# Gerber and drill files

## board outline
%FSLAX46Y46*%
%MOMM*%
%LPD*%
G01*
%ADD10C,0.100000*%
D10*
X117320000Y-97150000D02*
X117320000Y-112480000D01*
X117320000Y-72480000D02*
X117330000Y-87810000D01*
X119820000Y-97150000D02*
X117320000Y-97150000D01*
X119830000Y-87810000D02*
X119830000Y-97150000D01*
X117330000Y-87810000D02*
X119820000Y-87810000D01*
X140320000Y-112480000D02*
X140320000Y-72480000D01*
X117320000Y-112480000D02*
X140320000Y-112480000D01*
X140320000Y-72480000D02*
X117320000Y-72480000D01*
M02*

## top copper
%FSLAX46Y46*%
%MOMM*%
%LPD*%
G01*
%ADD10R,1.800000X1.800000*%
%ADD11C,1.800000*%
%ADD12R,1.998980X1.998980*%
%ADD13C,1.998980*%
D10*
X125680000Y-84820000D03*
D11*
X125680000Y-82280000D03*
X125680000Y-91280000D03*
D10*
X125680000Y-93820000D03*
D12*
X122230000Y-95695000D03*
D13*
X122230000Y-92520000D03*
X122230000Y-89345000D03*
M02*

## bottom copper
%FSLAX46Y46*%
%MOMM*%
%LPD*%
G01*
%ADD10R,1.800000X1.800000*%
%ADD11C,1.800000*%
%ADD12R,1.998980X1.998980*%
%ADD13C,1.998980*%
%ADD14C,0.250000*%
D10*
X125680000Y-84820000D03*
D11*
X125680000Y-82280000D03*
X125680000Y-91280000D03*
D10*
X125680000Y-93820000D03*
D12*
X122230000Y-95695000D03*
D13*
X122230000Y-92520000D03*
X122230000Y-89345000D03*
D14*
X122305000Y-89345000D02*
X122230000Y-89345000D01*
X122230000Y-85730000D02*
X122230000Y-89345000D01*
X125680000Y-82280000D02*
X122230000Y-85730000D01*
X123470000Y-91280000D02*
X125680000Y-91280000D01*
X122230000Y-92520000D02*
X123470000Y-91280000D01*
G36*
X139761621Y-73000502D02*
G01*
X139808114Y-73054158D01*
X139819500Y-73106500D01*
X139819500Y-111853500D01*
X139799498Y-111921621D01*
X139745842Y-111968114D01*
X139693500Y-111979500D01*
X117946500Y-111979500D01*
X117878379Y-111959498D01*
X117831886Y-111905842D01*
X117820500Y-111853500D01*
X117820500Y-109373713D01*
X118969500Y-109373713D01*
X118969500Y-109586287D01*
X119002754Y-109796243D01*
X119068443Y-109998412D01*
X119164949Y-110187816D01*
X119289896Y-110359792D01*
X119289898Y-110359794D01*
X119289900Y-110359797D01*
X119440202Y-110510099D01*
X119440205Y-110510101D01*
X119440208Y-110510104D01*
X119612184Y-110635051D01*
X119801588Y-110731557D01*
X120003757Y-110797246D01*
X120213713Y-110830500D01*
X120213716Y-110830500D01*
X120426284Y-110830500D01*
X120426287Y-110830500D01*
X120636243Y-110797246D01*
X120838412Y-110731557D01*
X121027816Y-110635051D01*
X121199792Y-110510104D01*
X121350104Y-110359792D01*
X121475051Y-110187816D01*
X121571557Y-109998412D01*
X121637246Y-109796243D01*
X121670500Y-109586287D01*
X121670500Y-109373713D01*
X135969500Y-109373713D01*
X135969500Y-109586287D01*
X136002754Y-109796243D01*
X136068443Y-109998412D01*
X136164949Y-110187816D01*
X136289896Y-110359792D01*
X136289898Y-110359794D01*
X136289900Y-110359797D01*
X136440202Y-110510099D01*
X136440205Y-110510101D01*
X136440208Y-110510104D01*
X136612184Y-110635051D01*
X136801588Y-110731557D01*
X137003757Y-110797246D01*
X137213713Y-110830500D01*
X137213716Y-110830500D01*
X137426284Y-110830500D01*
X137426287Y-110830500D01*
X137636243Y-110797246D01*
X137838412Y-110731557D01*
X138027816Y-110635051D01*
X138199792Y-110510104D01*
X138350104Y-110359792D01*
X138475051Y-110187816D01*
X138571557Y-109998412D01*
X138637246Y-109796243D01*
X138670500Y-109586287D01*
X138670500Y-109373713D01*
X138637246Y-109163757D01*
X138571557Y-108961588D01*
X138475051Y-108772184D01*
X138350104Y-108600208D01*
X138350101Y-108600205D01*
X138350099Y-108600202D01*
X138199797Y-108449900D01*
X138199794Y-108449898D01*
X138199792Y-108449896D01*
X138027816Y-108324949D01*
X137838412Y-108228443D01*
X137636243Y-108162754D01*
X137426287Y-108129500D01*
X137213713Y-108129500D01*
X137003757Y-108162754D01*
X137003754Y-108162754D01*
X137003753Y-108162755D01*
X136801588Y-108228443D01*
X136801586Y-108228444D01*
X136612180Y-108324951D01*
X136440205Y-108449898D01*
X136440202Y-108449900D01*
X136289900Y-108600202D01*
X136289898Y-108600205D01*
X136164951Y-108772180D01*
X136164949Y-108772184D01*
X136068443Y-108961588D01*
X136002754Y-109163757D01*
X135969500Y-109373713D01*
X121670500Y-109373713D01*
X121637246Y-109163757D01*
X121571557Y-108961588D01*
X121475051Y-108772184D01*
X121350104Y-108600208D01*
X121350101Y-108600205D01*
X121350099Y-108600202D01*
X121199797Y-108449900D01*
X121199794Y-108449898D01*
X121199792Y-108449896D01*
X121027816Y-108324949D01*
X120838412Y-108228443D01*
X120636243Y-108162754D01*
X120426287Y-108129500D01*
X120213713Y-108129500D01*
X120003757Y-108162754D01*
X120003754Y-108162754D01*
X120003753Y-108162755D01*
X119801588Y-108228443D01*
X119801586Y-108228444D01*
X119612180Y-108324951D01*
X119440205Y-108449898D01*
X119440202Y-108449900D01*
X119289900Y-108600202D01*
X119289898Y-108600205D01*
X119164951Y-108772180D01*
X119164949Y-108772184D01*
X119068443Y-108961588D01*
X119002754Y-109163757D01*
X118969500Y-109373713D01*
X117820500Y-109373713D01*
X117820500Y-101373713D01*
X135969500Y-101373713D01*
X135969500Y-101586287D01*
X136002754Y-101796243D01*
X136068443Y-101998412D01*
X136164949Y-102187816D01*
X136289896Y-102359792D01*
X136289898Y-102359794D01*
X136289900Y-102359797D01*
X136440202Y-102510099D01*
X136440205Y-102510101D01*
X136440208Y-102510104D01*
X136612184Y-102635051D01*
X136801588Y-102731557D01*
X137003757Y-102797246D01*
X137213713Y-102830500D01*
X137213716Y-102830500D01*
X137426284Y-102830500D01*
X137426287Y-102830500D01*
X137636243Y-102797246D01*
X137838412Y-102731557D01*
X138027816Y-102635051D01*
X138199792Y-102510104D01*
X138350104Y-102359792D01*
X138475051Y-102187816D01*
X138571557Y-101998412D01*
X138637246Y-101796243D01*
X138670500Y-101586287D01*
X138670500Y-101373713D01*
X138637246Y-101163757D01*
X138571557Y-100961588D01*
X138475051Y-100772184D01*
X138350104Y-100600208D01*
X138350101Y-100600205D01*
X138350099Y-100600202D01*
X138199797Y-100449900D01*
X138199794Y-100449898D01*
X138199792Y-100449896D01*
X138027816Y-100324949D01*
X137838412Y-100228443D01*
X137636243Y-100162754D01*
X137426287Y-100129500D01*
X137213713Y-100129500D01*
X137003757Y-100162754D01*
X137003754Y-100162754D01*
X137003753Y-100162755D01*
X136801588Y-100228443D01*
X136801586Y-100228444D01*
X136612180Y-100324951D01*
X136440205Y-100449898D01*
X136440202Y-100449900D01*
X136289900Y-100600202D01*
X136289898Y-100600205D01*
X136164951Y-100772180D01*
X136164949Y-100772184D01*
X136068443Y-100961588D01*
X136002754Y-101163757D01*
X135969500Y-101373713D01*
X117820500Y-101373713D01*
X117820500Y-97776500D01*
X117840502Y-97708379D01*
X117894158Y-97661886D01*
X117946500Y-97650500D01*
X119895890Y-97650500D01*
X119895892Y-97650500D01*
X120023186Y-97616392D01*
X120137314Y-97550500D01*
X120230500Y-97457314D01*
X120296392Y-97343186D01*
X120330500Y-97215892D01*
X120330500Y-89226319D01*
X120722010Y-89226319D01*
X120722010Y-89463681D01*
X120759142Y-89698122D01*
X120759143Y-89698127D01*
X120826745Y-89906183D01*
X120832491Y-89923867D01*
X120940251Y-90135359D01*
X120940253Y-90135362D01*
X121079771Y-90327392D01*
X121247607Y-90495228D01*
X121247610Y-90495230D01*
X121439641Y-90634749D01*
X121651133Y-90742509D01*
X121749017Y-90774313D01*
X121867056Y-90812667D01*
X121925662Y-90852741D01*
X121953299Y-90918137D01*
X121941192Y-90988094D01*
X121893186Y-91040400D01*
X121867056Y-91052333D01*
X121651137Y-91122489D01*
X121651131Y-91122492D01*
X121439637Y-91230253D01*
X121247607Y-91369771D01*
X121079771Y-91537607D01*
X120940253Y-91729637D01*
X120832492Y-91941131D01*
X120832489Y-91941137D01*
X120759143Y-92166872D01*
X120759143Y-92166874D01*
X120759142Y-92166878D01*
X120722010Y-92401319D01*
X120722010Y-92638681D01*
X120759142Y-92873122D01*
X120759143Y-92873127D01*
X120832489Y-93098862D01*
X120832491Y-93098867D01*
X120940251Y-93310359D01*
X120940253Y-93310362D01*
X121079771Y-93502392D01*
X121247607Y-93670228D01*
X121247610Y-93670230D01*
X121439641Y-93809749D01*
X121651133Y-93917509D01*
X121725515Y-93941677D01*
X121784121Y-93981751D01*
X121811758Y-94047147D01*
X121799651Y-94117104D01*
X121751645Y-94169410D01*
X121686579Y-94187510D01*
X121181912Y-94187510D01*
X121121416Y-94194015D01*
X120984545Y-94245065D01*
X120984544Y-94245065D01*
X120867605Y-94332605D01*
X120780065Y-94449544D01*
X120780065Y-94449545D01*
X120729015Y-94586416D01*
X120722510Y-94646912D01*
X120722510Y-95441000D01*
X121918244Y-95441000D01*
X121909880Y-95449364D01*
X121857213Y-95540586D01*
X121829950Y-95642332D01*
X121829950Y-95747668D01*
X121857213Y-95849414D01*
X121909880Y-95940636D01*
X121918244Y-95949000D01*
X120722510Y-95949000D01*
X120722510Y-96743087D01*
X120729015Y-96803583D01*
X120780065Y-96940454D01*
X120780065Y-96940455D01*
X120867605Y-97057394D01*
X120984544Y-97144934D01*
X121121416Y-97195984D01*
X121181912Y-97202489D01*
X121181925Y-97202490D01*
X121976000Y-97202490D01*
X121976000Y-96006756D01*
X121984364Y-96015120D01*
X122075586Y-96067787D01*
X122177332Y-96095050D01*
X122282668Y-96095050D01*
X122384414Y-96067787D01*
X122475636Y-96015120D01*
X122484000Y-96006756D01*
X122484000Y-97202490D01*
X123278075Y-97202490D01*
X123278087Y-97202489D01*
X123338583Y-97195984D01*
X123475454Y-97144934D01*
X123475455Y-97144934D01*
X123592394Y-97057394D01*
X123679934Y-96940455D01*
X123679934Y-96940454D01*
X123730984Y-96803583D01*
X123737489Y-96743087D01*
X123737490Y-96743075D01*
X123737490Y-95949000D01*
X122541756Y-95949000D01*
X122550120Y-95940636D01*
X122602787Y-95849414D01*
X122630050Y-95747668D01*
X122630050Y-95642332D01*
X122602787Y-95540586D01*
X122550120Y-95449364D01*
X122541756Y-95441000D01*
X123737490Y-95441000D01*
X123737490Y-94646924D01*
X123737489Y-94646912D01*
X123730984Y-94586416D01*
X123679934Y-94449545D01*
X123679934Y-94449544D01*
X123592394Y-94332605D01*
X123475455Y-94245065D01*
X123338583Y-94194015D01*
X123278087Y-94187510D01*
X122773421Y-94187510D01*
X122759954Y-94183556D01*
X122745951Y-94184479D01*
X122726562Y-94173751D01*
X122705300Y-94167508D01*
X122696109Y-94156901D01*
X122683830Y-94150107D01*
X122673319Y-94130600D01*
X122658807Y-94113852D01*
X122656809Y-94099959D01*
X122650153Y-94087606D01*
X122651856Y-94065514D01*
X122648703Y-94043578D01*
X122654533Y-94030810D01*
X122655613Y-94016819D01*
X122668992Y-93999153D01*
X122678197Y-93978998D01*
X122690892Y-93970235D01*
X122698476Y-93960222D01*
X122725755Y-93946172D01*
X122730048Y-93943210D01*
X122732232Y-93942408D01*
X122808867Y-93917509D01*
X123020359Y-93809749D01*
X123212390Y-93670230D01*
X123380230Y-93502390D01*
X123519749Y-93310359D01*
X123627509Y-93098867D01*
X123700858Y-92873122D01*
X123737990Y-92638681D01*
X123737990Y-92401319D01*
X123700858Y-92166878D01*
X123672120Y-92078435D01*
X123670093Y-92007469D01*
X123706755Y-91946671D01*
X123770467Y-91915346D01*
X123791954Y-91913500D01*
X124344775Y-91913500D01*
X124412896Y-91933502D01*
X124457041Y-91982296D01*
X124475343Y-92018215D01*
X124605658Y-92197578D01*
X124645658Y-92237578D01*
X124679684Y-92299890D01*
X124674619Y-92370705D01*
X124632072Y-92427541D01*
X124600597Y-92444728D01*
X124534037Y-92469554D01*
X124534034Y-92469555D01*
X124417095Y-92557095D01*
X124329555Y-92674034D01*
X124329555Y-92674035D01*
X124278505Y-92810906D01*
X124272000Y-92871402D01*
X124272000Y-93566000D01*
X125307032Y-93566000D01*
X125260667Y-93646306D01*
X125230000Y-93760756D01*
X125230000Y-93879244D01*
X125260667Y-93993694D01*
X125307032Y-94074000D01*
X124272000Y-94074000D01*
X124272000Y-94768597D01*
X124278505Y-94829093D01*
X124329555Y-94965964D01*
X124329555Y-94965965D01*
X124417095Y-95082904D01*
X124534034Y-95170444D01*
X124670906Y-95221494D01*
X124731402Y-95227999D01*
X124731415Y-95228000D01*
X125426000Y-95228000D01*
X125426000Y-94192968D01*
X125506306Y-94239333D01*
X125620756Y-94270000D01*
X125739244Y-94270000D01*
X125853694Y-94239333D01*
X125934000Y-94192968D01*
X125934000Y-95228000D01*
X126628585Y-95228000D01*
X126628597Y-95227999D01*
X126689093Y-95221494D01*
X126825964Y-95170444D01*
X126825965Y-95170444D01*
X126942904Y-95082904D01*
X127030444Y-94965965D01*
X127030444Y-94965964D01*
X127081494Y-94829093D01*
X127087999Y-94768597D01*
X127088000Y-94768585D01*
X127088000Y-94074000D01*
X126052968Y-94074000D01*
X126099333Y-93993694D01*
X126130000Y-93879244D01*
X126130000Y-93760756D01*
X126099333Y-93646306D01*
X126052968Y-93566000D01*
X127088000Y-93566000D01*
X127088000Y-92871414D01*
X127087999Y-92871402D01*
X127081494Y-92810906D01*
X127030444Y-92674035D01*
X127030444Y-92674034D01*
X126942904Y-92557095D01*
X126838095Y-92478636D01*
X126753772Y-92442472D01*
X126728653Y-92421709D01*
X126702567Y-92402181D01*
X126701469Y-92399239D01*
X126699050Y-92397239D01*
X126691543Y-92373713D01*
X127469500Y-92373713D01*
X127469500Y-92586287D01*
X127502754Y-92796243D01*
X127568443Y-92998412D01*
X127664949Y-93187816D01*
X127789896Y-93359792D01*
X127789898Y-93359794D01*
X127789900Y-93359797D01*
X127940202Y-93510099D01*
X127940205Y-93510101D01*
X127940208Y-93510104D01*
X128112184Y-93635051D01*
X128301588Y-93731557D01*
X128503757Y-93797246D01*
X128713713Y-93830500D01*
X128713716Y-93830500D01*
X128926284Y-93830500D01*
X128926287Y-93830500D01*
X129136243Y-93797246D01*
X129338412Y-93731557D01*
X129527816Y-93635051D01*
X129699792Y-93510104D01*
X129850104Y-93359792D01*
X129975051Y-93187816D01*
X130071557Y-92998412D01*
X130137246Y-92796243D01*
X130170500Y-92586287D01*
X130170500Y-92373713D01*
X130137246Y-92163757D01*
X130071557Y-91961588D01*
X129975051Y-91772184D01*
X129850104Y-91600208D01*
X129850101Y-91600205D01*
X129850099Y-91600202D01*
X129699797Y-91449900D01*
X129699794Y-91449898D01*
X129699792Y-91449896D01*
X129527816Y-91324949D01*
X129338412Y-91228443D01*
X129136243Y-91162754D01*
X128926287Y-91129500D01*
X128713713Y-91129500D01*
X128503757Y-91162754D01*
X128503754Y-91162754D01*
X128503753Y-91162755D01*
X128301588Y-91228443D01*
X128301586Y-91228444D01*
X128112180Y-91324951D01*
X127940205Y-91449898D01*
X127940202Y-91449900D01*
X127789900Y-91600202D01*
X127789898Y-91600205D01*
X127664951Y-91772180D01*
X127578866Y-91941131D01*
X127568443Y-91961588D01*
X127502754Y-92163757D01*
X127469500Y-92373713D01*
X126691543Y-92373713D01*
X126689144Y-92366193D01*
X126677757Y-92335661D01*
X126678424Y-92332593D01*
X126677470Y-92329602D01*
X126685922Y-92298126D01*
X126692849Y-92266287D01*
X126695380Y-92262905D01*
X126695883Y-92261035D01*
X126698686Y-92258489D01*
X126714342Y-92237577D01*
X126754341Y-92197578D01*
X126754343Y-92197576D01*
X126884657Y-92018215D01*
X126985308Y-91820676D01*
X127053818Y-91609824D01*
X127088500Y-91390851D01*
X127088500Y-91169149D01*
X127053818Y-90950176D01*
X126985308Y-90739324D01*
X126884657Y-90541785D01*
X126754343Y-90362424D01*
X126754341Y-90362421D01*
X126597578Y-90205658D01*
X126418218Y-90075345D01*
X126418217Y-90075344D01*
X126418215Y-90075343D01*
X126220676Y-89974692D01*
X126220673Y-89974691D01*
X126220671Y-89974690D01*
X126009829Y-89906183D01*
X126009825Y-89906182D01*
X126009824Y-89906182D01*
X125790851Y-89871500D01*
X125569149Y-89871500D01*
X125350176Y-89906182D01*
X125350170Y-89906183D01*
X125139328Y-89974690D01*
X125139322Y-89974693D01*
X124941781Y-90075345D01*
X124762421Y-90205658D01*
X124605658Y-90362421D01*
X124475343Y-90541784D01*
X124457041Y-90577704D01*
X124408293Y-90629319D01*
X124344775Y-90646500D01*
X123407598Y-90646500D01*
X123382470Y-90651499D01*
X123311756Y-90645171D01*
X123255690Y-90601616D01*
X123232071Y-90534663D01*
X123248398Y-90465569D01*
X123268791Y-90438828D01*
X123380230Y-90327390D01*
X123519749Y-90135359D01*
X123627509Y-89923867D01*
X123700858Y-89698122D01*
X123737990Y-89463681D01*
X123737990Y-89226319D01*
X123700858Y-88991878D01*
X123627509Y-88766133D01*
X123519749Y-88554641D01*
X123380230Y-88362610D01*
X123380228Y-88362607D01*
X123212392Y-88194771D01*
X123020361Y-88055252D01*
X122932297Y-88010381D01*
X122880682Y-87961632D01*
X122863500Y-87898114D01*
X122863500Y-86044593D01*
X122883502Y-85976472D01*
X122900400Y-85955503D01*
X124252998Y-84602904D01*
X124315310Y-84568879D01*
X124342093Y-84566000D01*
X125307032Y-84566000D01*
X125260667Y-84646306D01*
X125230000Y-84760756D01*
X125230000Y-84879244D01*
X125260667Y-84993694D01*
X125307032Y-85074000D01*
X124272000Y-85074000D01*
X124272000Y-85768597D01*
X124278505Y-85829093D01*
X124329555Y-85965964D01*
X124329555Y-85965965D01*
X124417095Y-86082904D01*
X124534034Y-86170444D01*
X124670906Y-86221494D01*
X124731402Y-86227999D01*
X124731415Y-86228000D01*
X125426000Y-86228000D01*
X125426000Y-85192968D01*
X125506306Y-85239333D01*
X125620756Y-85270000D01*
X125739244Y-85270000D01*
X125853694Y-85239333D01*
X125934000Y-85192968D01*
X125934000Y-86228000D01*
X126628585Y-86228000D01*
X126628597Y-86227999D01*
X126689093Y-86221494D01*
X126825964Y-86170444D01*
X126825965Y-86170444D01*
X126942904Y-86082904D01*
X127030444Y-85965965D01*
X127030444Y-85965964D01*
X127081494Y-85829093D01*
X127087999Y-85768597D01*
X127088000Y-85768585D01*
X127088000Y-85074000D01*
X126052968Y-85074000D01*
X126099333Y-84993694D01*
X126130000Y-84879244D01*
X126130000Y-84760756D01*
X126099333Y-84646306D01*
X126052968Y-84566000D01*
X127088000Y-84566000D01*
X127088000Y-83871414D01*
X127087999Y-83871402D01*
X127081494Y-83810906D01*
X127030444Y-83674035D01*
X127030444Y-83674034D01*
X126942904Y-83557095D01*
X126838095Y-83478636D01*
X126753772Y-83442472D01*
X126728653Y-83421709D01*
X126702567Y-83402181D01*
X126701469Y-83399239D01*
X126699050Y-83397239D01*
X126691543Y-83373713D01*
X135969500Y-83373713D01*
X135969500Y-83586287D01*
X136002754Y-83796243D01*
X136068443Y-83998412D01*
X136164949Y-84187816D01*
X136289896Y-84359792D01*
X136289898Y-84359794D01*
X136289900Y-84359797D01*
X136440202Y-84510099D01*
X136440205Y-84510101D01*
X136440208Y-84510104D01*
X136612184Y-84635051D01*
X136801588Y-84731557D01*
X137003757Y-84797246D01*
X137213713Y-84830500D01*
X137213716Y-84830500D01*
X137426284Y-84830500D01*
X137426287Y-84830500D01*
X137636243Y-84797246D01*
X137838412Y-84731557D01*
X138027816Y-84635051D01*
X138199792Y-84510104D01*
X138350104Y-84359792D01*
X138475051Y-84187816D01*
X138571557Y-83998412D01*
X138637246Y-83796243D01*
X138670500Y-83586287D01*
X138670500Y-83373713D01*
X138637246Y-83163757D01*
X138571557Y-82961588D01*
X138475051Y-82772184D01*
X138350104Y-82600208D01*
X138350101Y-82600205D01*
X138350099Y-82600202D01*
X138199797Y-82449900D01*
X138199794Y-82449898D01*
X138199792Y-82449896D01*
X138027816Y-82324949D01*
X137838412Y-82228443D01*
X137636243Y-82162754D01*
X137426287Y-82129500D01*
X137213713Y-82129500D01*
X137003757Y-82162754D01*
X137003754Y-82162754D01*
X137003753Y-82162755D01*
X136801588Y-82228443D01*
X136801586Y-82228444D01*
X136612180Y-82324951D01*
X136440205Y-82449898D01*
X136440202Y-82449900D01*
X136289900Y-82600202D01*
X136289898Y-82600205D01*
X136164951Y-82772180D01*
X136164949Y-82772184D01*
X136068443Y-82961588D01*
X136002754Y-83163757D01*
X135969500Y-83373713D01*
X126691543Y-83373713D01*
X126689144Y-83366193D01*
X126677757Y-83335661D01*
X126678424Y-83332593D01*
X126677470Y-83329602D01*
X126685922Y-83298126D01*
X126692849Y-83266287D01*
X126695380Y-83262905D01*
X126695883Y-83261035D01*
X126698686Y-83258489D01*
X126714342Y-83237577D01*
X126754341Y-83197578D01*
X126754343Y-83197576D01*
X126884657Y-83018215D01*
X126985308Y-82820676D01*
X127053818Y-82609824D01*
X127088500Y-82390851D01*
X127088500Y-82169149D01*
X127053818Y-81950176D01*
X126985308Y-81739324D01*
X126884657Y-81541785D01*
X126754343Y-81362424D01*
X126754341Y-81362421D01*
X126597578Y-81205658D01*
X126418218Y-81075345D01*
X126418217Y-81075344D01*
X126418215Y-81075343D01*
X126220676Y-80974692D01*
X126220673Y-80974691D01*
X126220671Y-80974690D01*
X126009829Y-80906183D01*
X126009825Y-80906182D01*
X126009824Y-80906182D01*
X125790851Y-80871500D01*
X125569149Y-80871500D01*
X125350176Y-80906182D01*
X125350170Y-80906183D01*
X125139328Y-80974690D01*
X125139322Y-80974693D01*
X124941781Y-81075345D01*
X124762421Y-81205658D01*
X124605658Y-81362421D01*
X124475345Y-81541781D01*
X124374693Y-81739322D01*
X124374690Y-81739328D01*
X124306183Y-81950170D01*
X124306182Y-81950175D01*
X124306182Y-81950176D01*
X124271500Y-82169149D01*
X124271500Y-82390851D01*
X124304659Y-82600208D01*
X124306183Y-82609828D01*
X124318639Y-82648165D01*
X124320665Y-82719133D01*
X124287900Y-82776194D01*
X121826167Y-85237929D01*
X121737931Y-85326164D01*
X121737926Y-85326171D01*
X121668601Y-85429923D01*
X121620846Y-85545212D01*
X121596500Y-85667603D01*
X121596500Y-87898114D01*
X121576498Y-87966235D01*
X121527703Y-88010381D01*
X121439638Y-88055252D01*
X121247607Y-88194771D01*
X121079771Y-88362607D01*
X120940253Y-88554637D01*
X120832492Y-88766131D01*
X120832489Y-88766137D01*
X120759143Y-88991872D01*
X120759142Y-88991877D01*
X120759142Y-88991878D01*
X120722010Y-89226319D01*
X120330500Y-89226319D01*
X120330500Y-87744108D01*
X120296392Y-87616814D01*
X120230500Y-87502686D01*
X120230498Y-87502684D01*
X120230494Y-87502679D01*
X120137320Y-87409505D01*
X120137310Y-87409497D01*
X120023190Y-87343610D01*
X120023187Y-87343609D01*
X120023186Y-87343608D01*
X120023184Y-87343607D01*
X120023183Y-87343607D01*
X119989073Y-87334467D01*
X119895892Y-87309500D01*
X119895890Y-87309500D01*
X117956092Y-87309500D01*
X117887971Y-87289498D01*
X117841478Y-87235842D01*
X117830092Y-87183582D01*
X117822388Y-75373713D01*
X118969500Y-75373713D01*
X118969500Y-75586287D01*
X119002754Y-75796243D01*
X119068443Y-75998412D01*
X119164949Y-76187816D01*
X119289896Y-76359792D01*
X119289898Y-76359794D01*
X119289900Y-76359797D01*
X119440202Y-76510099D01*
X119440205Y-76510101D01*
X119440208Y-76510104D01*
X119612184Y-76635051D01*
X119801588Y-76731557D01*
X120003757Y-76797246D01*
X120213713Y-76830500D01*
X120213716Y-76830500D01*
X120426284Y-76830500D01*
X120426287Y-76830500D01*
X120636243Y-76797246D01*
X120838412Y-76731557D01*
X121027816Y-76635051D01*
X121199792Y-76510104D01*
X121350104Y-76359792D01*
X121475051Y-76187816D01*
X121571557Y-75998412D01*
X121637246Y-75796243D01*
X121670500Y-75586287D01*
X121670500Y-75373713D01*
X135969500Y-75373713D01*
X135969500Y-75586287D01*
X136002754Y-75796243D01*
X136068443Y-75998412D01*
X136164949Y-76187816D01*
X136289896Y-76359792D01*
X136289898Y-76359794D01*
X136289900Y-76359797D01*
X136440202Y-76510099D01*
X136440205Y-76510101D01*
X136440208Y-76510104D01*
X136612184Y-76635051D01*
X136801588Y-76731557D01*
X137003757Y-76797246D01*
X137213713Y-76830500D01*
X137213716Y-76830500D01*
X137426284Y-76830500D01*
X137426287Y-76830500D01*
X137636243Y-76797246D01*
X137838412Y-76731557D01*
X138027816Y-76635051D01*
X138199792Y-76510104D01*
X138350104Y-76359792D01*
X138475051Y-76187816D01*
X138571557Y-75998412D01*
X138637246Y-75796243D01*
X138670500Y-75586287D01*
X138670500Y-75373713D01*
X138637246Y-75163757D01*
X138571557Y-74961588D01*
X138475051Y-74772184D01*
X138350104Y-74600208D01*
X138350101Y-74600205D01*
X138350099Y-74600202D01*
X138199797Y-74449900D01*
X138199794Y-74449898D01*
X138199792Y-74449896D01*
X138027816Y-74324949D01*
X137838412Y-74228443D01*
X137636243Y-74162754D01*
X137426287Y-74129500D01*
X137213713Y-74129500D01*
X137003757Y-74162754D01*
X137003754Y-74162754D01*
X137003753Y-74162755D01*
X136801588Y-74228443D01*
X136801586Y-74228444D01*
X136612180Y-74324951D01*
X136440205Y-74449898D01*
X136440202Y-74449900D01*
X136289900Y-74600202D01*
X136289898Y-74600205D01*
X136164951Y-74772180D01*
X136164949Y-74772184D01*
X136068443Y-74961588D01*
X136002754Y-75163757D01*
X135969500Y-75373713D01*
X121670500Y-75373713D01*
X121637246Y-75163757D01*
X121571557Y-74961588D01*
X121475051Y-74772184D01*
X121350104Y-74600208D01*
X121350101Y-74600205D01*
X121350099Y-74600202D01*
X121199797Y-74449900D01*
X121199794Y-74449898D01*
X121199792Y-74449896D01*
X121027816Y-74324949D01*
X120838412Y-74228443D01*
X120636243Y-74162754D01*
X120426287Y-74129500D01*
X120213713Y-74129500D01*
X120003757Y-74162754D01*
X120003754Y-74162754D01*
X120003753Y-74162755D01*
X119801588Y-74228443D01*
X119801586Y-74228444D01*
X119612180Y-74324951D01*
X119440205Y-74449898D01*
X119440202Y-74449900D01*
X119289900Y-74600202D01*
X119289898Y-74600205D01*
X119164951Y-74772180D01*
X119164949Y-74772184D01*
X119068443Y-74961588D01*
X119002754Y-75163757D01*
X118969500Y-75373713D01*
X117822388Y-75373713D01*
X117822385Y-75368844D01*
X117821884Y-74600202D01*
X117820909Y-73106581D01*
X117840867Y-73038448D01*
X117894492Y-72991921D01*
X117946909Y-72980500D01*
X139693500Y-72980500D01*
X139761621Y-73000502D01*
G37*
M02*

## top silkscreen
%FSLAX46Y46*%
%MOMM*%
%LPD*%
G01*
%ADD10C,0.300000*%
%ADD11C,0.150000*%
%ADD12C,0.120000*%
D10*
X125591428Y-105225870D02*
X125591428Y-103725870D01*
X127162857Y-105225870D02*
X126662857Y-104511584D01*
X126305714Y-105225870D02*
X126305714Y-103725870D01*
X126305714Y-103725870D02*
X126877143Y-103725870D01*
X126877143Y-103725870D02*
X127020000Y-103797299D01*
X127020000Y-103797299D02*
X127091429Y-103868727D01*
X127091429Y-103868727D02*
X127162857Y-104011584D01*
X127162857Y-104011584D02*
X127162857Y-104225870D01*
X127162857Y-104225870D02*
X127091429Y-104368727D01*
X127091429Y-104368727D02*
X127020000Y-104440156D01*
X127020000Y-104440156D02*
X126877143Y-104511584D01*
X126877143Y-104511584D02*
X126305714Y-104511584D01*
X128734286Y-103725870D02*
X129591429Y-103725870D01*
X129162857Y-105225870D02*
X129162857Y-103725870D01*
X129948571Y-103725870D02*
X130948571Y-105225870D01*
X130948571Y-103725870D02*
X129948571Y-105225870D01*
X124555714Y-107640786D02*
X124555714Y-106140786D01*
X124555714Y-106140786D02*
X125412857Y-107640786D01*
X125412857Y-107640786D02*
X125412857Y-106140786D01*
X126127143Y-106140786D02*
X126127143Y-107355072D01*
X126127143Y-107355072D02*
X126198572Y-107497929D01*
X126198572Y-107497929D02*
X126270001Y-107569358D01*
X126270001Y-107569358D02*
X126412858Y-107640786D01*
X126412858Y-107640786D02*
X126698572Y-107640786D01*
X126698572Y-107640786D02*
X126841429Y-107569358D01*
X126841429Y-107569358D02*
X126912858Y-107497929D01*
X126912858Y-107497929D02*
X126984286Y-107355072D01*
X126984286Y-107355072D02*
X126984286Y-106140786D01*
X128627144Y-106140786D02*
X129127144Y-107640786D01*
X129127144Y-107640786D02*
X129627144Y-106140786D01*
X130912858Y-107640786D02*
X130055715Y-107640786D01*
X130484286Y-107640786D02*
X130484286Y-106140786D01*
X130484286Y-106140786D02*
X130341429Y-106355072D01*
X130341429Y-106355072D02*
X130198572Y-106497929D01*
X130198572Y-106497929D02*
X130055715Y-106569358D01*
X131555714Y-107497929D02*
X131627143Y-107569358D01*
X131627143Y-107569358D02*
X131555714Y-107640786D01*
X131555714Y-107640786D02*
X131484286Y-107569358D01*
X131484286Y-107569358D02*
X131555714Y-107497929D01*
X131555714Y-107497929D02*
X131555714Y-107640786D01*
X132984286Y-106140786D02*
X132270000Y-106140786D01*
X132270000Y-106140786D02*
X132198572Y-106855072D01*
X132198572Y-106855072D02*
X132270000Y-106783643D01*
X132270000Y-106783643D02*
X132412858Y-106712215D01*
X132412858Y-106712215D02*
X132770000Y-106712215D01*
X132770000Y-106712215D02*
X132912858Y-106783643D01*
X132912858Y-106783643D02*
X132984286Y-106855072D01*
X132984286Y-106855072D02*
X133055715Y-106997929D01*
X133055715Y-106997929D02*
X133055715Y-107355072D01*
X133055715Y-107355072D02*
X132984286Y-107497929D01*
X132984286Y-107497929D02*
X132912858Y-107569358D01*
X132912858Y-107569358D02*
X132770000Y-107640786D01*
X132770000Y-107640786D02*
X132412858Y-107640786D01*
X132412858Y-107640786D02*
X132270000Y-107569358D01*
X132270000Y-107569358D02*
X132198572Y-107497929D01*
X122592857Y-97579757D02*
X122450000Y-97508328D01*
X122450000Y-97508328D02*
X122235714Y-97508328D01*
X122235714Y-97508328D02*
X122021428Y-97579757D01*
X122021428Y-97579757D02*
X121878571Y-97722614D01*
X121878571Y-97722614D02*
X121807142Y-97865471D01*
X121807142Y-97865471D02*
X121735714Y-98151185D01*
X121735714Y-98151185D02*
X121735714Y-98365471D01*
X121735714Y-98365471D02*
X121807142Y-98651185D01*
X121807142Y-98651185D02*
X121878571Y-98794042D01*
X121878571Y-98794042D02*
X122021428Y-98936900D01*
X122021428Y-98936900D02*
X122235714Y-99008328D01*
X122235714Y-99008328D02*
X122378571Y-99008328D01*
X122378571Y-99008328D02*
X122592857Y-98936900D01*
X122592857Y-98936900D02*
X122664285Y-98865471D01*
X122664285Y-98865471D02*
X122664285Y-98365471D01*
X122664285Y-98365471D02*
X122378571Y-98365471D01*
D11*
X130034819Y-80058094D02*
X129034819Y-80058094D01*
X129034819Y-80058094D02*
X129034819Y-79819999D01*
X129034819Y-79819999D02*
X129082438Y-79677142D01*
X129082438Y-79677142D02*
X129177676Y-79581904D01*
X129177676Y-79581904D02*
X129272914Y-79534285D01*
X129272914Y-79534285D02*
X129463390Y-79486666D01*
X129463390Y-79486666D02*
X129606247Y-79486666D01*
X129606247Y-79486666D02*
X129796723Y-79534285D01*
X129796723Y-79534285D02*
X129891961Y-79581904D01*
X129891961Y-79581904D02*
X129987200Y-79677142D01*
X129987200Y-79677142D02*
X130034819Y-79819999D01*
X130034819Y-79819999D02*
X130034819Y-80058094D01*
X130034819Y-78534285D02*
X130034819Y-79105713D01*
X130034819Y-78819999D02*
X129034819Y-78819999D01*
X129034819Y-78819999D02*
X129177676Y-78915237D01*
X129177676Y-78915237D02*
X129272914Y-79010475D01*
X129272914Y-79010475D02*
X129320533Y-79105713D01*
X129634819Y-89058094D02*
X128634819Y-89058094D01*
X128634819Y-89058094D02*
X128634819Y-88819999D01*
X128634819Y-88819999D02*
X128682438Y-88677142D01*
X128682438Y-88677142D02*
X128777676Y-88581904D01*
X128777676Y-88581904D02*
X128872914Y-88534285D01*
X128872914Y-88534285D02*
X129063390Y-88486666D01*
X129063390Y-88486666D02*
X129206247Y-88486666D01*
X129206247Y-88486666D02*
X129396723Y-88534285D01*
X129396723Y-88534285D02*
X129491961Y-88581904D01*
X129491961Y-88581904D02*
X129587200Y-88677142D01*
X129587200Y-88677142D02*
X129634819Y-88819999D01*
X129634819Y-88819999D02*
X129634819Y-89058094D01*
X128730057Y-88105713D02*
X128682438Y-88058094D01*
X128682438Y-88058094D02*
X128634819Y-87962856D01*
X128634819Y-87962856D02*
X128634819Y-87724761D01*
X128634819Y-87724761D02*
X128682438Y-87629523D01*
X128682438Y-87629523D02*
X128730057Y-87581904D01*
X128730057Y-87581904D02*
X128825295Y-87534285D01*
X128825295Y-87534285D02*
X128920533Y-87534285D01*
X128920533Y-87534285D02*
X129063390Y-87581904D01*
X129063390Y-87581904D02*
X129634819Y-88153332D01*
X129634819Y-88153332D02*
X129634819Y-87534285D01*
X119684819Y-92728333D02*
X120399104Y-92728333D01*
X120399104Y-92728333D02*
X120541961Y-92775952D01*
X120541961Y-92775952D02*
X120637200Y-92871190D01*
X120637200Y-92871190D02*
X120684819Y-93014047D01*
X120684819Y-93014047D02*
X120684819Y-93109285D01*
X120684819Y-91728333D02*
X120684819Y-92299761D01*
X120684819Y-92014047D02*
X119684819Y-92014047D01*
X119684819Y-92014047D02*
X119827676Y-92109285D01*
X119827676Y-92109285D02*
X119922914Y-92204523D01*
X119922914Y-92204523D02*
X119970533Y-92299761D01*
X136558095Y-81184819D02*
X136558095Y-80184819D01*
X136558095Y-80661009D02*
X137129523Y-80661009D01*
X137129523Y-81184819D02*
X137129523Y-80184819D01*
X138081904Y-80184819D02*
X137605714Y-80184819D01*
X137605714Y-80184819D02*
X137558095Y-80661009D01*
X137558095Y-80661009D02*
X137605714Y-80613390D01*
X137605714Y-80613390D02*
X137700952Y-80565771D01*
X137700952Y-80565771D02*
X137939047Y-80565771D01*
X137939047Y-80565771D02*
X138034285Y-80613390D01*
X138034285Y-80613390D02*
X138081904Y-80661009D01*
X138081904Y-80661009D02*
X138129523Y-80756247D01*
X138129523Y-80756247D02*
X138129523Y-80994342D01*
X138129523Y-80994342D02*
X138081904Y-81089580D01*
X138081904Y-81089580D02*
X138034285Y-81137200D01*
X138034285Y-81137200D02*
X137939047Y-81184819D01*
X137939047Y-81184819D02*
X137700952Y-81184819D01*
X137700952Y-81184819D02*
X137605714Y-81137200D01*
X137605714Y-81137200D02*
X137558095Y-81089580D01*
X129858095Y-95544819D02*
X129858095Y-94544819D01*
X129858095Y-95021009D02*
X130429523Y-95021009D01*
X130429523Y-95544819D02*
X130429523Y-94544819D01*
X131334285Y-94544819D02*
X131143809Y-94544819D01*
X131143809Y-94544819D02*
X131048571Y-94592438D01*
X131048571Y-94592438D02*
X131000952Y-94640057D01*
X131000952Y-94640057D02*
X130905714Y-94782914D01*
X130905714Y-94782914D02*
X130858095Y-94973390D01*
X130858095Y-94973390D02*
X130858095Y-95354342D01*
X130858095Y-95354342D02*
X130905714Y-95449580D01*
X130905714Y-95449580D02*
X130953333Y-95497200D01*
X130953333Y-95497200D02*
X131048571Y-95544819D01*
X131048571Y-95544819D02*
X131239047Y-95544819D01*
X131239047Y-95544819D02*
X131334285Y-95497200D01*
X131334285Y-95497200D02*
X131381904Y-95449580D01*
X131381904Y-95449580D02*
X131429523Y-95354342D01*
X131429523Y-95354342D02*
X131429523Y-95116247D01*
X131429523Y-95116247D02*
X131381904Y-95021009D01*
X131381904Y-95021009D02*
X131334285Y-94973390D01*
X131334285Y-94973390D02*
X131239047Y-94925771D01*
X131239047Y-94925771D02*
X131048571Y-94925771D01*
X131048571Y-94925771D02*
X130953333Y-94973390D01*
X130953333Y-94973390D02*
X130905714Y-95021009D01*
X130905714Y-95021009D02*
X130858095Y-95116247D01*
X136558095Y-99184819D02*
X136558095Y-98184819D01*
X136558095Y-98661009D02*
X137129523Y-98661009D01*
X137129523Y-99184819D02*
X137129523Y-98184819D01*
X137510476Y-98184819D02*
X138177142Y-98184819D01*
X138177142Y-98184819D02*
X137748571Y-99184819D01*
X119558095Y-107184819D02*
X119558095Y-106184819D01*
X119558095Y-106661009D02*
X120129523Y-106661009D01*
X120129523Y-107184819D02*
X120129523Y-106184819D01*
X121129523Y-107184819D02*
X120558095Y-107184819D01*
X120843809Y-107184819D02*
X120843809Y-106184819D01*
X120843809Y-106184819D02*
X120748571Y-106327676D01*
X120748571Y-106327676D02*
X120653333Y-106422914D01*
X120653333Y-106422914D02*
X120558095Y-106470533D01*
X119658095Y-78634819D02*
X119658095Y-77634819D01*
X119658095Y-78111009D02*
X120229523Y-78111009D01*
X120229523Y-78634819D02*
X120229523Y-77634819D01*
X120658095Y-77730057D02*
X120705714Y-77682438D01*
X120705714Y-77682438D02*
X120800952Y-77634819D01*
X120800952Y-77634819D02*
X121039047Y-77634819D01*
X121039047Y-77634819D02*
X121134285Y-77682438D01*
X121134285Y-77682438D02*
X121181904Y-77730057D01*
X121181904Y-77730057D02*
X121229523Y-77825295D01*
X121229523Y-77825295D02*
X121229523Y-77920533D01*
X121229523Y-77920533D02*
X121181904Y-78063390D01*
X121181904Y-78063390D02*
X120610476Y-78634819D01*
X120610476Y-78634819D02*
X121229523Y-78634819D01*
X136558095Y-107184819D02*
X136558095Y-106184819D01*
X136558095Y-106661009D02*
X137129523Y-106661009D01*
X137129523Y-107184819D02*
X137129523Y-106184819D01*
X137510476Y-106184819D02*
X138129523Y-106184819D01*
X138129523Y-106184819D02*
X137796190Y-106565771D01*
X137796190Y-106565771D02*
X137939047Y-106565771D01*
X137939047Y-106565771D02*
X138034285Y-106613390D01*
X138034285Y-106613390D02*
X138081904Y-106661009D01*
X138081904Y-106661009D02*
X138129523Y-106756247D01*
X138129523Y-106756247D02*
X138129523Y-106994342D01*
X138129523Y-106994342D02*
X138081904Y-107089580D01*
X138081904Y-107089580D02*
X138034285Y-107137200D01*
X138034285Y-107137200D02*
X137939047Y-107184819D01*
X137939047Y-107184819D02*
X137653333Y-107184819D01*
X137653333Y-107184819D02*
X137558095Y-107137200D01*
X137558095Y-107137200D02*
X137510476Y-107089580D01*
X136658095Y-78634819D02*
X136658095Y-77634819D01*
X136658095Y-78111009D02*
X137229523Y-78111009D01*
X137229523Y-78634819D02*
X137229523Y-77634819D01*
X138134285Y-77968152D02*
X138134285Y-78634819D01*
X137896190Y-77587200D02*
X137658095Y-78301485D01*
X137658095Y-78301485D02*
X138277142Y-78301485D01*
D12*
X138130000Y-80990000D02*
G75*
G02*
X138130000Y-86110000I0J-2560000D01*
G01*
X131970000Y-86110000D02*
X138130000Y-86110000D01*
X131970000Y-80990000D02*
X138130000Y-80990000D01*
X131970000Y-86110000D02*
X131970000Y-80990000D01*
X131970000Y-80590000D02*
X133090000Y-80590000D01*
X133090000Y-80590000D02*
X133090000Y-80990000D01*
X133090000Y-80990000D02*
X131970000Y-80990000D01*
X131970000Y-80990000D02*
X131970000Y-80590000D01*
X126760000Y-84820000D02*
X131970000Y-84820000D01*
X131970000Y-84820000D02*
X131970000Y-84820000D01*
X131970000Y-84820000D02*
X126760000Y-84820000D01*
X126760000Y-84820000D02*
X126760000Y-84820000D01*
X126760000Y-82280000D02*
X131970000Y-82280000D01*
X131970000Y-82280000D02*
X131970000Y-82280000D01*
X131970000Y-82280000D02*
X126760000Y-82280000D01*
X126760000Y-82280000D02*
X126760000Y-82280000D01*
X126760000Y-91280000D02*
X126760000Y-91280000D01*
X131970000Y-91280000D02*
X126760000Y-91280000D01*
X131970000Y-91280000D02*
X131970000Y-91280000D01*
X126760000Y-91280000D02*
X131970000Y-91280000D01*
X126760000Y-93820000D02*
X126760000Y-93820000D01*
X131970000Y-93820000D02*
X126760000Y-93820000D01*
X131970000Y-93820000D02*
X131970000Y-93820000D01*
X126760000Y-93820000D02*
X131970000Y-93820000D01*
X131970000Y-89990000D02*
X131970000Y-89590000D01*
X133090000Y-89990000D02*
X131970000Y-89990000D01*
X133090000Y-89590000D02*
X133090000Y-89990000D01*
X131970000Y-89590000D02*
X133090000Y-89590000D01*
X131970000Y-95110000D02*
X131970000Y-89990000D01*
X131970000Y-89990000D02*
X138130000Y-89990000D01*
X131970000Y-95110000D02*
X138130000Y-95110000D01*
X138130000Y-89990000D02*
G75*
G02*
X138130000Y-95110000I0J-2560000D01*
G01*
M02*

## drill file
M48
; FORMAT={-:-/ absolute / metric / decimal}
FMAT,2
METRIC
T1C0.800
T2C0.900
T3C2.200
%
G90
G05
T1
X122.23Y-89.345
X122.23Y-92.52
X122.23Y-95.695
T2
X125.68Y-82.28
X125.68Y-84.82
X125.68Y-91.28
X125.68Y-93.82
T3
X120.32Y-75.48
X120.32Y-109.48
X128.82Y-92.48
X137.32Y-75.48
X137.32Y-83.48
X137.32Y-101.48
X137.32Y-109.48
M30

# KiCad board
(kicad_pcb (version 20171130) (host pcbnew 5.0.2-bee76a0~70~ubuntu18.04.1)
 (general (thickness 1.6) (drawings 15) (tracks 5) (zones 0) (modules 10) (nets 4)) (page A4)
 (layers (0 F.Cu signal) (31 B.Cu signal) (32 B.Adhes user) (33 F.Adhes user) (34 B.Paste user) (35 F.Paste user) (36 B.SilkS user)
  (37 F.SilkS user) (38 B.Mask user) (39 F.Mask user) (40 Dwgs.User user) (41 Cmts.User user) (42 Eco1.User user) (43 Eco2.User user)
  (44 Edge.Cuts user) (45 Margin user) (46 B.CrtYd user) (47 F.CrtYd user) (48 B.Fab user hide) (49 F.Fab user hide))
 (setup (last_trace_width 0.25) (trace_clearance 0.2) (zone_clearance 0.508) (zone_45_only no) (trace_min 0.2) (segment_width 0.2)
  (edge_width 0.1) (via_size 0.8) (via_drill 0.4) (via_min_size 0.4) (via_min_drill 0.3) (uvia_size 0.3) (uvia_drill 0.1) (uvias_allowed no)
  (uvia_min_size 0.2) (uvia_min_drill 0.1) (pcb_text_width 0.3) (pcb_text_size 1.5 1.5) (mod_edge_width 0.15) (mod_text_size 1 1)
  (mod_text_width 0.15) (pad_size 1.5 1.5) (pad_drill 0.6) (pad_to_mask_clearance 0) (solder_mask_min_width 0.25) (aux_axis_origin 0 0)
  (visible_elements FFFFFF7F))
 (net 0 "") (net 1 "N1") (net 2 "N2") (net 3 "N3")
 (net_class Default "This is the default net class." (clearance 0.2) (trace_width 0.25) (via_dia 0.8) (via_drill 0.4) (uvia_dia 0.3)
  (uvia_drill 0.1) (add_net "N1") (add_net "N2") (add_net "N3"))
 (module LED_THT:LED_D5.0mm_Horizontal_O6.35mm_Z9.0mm (layer F.Cu) (at 125.68 84.82 90)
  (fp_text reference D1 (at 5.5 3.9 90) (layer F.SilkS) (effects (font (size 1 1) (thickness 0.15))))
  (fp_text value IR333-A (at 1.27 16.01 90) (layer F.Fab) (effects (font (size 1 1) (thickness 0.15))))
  (fp_arc (start 1.27 12.45) (end -1.29 12.45) (angle -180) (layer F.SilkS) (width 0.12))
  (fp_line (start -1.29 6.29) (end -1.29 12.45) (layer F.SilkS) (width 0.12))
  (fp_line (start 3.83 6.29) (end 3.83 12.45) (layer F.SilkS) (width 0.12))
  (fp_line (start -1.29 6.29) (end 3.83 6.29) (layer F.SilkS) (width 0.12))
  (fp_line (start 4.23 6.29) (end 4.23 7.41) (layer F.SilkS) (width 0.12))
  (fp_line (start 4.23 7.41) (end 3.83 7.41) (layer F.SilkS) (width 0.12))
  (fp_line (start 3.83 7.41) (end 3.83 6.29) (layer F.SilkS) (width 0.12))
  (fp_line (start 3.83 6.29) (end 4.23 6.29) (layer F.SilkS) (width 0.12))
  (fp_line (start 0 1.08) (end 0 6.29) (layer F.SilkS) (width 0.12))
  (fp_line (start 0 6.29) (end 0 6.29) (layer F.SilkS) (width 0.12))
  (fp_line (start 0 6.29) (end 0 1.08) (layer F.SilkS) (width 0.12))
  (fp_line (start 0 1.08) (end 0 1.08) (layer F.SilkS) (width 0.12))
  (fp_line (start 2.54 1.08) (end 2.54 6.29) (layer F.SilkS) (width 0.12))
  (fp_line (start 2.54 6.29) (end 2.54 6.29) (layer F.SilkS) (width 0.12))
  (fp_line (start 2.54 6.29) (end 2.54 1.08) (layer F.SilkS) (width 0.12))
  (fp_line (start 2.54 1.08) (end 2.54 1.08) (layer F.SilkS) (width 0.12))
  (pad 1 thru_hole rect (at 0 0 90) (size 1.8 1.8) (drill 0.9) (layers *.Cu *.Mask) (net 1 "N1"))
  (pad 2 thru_hole circle (at 2.54 0 90) (size 1.8 1.8) (drill 0.9) (layers *.Cu *.Mask) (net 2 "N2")))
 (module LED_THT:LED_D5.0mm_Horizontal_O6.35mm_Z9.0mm (layer F.Cu) (at 125.68 93.82 90)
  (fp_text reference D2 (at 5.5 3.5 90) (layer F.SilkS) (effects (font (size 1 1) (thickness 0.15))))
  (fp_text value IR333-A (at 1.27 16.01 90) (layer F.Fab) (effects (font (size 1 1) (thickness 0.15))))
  (fp_line (start 2.54 1.08) (end 2.54 1.08) (layer F.SilkS) (width 0.12))
  (fp_line (start 2.54 6.29) (end 2.54 1.08) (layer F.SilkS) (width 0.12))
  (fp_line (start 2.54 6.29) (end 2.54 6.29) (layer F.SilkS) (width 0.12))
  (fp_line (start 2.54 1.08) (end 2.54 6.29) (layer F.SilkS) (width 0.12))
  (fp_line (start 0 1.08) (end 0 1.08) (layer F.SilkS) (width 0.12))
  (fp_line (start 0 6.29) (end 0 1.08) (layer F.SilkS) (width 0.12))
  (fp_line (start 0 6.29) (end 0 6.29) (layer F.SilkS) (width 0.12))
  (fp_line (start 0 1.08) (end 0 6.29) (layer F.SilkS) (width 0.12))
  (fp_line (start 3.83 6.29) (end 4.23 6.29) (layer F.SilkS) (width 0.12))
  (fp_line (start 3.83 7.41) (end 3.83 6.29) (layer F.SilkS) (width 0.12))
  (fp_line (start 4.23 7.41) (end 3.83 7.41) (layer F.SilkS) (width 0.12))
  (fp_line (start 4.23 6.29) (end 4.23 7.41) (layer F.SilkS) (width 0.12))
  (fp_line (start -1.29 6.29) (end 3.83 6.29) (layer F.SilkS) (width 0.12))
  (fp_line (start 3.83 6.29) (end 3.83 12.45) (layer F.SilkS) (width 0.12))
  (fp_line (start -1.29 6.29) (end -1.29 12.45) (layer F.SilkS) (width 0.12))
  (fp_arc (start 1.27 12.45) (end -1.29 12.45) (angle -180) (layer F.SilkS) (width 0.12))
  (pad 2 thru_hole circle (at 2.54 0 90) (size 1.8 1.8) (drill 0.9) (layers *.Cu *.Mask) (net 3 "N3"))
  (pad 1 thru_hole rect (at 0 0 90) (size 1.8 1.8) (drill 0.9) (layers *.Cu *.Mask) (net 1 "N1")))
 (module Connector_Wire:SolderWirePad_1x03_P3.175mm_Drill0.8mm (layer F.Cu) (at 122.23 95.695 90)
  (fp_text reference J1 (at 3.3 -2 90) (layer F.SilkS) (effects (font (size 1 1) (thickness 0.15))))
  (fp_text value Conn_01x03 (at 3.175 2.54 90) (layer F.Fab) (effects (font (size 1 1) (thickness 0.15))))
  (pad 1 thru_hole rect (at 0 0 90) (size 1.99898 1.99898) (drill 0.8001) (layers *.Cu *.Mask) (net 1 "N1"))
  (pad 2 thru_hole circle (at 3.175 0 90) (size 1.99898 1.99898) (drill 0.8001) (layers *.Cu *.Mask) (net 3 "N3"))
  (pad 3 thru_hole circle (at 6.35 0 90) (size 1.99898 1.99898) (drill 0.8001) (layers *.Cu *.Mask) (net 2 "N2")))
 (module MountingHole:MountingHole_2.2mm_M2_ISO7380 (layer F.Cu) (at 137.32 83.48)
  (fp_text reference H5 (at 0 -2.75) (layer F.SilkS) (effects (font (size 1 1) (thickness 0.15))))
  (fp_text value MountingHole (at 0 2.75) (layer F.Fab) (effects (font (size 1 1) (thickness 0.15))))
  (pad 1 np_thru_hole circle (at 0 0) (size 2.2 2.2) (drill 2.2) (layers *.Cu *.Mask)))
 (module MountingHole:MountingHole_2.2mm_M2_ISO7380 (layer F.Cu) (at 128.82 92.48)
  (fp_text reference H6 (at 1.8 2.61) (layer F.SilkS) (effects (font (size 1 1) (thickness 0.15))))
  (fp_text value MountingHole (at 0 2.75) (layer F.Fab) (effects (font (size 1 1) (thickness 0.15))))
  (pad 1 np_thru_hole circle (at 0 0) (size 2.2 2.2) (drill 2.2) (layers *.Cu *.Mask)))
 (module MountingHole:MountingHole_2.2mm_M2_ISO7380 (layer F.Cu) (at 137.32 101.48)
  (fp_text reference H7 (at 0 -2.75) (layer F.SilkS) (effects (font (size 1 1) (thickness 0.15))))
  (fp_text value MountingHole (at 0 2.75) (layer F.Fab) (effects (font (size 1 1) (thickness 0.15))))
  (pad 1 np_thru_hole circle (at 0 0) (size 2.2 2.2) (drill 2.2) (layers *.Cu *.Mask)))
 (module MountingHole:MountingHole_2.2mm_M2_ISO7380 (layer F.Cu) (at 120.32 109.48)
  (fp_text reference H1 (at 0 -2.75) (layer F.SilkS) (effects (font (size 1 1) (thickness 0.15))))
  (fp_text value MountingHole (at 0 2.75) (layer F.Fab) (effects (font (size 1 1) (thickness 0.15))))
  (pad 1 np_thru_hole circle (at 0 0) (size 2.2 2.2) (drill 2.2) (layers *.Cu *.Mask)))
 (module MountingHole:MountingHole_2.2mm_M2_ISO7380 (layer F.Cu) (at 120.32 75.48)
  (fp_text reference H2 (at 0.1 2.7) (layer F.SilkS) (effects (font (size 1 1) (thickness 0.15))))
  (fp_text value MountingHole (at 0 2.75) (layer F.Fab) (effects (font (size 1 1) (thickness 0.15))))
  (pad 1 np_thru_hole circle (at 0 0) (size 2.2 2.2) (drill 2.2) (layers *.Cu *.Mask)))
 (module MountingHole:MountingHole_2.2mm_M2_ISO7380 (layer F.Cu) (at 137.32 109.48)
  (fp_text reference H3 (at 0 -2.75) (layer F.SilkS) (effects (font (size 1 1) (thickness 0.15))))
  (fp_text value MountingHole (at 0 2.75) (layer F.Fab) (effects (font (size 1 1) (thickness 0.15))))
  (pad 1 np_thru_hole circle (at 0 0) (size 2.2 2.2) (drill 2.2) (layers *.Cu *.Mask)))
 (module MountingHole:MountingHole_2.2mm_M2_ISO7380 (layer F.Cu) (at 137.32 75.48)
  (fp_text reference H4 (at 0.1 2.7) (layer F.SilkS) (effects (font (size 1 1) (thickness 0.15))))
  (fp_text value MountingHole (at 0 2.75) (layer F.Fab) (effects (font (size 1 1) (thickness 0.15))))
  (pad 1 np_thru_hole circle (at 0 0) (size 2.2 2.2) (drill 2.2) (layers *.Cu *.Mask)))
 (gr_line (start 117.32 97.15) (end 117.32 112.48) (layer Edge.Cuts) (width 0.1))
 (gr_line (start 117.32 72.48) (end 117.33 87.81) (layer Edge.Cuts) (width 0.1))
 (gr_line (start 119.82 97.15) (end 117.32 97.15) (layer Edge.Cuts) (width 0.1))
 (gr_line (start 119.83 87.81) (end 119.83 97.15) (layer Edge.Cuts) (width 0.1))
 (gr_line (start 117.33 87.81) (end 119.82 87.81) (layer Edge.Cuts) (width 0.1))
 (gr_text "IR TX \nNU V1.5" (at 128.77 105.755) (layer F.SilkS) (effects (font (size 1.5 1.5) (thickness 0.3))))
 (gr_line (start 140.32 112.48) (end 140.32 72.48) (layer Edge.Cuts) (width 0.1))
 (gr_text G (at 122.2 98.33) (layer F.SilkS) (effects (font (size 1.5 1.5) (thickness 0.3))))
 (gr_line (start 117.32 112.48) (end 140.32 112.48) (layer Edge.Cuts) (width 0.1))
 (gr_line (start 140.32 72.48) (end 117.32 72.48) (layer Edge.Cuts) (width 0.1))
 (segment (start 122.305 89.345) (end 122.23 89.345) (width 0.25) (layer B.Cu) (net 2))
 (segment (start 122.23 85.73) (end 122.23 89.345) (width 0.25) (layer B.Cu) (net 2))
 (segment (start 125.68 82.28) (end 122.23 85.73) (width 0.25) (layer B.Cu) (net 2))
 (segment (start 123.47 91.28) (end 125.68 91.28) (width 0.25) (layer B.Cu) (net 3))
 (segment (start 122.23 92.52) (end 123.47 91.28) (width 0.25) (layer B.Cu) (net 3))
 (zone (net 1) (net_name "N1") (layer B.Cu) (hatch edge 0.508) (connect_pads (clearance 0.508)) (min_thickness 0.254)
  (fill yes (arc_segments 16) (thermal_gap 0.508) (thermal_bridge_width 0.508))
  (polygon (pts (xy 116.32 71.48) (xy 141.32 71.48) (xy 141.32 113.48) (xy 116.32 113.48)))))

